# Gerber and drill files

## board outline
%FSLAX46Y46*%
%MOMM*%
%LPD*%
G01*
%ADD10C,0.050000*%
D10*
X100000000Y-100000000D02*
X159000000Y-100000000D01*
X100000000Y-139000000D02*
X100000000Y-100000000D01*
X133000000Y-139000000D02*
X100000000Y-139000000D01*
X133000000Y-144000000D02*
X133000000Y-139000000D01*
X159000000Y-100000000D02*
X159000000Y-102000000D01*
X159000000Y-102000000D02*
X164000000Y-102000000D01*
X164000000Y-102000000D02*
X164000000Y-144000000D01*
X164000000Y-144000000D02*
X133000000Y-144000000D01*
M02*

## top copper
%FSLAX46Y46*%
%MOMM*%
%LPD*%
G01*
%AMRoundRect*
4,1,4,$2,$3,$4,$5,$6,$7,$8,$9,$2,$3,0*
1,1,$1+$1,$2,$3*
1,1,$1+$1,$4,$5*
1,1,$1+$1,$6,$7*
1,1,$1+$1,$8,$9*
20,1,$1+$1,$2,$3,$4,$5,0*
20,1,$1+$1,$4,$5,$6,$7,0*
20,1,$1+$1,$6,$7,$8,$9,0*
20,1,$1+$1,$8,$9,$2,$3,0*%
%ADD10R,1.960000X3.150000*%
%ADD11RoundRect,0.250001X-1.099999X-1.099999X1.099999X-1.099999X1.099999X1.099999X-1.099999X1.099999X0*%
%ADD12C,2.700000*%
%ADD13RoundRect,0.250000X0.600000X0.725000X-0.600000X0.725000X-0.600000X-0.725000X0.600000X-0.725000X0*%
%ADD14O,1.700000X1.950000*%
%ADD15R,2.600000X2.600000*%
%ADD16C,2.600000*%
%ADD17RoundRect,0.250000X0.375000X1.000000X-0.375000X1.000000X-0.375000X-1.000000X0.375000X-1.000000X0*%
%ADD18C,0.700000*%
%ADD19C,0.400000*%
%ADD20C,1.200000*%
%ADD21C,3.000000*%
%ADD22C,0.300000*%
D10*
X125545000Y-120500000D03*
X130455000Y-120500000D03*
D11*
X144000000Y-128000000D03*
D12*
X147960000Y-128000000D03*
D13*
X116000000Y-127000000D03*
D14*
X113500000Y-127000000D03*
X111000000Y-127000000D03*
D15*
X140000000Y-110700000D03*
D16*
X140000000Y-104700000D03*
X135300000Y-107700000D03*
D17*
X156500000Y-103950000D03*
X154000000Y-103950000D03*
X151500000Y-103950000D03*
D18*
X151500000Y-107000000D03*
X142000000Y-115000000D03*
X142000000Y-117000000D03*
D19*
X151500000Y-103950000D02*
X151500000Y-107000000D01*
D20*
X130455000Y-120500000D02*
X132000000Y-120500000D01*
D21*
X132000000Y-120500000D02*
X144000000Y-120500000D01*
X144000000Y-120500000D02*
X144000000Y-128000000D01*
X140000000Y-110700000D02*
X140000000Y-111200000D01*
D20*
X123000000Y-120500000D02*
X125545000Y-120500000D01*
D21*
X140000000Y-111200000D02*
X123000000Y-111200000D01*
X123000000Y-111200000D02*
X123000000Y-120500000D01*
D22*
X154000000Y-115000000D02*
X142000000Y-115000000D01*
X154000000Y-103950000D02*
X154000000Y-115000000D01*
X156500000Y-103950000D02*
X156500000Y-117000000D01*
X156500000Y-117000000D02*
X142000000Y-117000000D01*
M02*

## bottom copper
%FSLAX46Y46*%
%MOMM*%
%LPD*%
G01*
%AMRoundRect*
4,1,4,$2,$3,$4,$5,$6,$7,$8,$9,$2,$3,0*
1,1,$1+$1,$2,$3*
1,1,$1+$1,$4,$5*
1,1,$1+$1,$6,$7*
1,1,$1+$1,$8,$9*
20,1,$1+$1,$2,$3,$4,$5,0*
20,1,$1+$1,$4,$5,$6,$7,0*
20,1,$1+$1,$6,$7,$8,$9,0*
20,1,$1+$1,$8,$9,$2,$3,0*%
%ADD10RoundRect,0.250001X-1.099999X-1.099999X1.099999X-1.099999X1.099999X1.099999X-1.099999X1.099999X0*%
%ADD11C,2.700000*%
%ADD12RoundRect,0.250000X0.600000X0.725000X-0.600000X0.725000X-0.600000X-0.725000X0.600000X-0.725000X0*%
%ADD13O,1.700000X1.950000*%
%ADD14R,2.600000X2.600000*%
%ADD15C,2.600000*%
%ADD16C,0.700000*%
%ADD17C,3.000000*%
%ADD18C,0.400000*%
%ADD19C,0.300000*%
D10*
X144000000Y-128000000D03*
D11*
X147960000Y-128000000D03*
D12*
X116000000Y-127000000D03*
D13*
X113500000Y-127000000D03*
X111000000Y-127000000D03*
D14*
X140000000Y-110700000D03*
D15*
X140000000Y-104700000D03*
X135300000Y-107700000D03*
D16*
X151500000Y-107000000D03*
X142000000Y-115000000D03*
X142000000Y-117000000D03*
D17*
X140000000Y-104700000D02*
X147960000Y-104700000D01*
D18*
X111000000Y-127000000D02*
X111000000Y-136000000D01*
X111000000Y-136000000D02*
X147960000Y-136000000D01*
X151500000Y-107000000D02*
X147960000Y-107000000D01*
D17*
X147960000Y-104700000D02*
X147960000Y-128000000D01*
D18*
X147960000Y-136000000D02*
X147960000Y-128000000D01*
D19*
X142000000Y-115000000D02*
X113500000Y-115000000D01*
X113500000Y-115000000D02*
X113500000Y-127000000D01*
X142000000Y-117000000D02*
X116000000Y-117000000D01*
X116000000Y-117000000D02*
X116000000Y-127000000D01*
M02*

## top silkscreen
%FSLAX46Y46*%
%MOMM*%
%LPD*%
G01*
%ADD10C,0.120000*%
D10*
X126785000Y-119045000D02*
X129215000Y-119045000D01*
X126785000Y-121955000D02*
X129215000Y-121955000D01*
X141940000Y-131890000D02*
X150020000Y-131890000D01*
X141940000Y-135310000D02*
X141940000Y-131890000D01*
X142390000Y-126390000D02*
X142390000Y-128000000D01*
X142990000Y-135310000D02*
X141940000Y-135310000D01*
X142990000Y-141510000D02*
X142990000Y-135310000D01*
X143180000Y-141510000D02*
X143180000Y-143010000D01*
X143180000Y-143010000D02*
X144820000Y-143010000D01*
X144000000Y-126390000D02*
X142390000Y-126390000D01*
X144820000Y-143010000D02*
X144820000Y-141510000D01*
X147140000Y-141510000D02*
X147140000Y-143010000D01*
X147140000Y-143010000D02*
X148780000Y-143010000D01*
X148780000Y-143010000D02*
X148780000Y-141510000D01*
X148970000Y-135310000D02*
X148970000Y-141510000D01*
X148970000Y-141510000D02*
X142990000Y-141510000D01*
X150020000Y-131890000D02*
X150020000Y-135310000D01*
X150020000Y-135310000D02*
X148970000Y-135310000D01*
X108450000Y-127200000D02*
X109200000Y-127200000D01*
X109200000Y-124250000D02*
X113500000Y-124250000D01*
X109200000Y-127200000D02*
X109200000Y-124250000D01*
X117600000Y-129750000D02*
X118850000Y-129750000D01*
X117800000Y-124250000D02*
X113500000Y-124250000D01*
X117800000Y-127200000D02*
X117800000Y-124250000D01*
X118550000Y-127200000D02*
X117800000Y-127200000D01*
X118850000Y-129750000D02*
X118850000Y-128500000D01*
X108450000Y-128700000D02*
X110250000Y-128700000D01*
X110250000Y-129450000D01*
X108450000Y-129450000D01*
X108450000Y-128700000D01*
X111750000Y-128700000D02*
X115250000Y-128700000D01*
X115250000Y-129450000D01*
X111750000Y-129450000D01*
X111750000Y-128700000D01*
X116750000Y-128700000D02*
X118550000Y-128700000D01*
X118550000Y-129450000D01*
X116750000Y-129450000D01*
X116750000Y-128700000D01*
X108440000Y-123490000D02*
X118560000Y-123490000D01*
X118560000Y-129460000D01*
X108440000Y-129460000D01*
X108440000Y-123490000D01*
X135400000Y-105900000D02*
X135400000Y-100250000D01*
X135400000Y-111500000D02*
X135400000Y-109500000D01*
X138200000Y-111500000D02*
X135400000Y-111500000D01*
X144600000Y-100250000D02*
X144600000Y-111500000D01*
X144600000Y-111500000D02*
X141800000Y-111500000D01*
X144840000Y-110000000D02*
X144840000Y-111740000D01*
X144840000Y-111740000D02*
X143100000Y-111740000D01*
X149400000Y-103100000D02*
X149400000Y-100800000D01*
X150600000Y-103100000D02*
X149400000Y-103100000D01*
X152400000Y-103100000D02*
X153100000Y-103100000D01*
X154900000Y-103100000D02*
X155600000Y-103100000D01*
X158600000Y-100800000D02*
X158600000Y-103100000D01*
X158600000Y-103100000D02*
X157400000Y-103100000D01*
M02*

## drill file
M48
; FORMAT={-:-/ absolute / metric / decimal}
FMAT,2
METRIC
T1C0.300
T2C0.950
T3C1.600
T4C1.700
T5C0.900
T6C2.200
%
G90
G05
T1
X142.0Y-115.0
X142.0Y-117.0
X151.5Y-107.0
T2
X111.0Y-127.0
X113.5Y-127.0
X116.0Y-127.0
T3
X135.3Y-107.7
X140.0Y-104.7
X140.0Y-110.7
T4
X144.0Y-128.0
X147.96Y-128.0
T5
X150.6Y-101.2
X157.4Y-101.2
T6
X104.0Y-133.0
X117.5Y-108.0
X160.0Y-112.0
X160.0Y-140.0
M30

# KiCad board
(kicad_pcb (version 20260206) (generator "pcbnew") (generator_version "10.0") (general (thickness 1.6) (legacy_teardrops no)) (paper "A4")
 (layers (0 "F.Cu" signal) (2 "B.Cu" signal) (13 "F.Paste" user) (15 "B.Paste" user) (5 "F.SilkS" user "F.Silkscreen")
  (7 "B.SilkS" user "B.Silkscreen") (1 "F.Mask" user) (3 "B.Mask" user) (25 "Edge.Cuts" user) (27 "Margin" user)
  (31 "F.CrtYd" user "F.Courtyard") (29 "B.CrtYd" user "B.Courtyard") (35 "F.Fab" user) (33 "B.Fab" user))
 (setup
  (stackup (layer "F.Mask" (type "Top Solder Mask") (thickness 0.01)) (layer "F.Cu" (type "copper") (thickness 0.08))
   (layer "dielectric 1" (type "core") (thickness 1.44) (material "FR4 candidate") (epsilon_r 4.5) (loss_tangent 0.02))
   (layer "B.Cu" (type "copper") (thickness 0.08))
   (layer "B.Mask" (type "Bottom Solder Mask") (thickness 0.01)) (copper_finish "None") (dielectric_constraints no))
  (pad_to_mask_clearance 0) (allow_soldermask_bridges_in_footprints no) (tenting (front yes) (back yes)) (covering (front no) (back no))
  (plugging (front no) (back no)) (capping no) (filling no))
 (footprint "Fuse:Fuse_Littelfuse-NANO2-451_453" (layer "F.Cu") (at 128 120.5)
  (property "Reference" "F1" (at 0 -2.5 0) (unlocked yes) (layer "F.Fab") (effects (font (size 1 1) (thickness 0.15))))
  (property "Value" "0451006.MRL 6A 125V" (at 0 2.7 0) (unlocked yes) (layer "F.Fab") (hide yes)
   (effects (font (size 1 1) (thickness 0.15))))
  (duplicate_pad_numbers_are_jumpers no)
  (fp_line (start -1.215 -1.455) (end 1.215 -1.455) (stroke (width 0.12) (type solid)) (layer "F.SilkS"))
  (fp_line (start -1.215 1.455) (end 1.215 1.455) (stroke (width 0.12) (type solid)) (layer "F.SilkS"))
  (pad "1" smd rect (at -2.455 0) (size 1.96 3.15) (layers "F.Cu" "F.Mask" "F.Paste") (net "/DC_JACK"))
  (pad "2" smd rect (at 2.455 0) (size 1.96 3.15) (layers "F.Cu" "F.Mask" "F.Paste") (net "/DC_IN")))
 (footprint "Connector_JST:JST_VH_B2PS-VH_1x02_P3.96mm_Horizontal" (layer "F.Cu") (at 144 128)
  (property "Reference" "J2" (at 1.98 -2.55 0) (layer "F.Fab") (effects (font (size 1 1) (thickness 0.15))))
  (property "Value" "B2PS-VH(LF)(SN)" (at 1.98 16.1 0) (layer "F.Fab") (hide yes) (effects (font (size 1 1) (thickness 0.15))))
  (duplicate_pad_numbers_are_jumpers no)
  (fp_line (start -2.06 3.89) (end 6.02 3.89) (stroke (width 0.12) (type solid)) (layer "F.SilkS"))
  (fp_line (start -2.06 7.31) (end -2.06 3.89) (stroke (width 0.12) (type solid)) (layer "F.SilkS"))
  (fp_line (start -1.61 -1.61) (end -1.61 0) (stroke (width 0.12) (type solid)) (layer "F.SilkS"))
  (fp_line (start -1.01 7.31) (end -2.06 7.31) (stroke (width 0.12) (type solid)) (layer "F.SilkS"))
  (fp_line (start -1.01 13.51) (end -1.01 7.31) (stroke (width 0.12) (type solid)) (layer "F.SilkS"))
  (fp_line (start -0.82 13.51) (end -0.82 15.01) (stroke (width 0.12) (type solid)) (layer "F.SilkS"))
  (fp_line (start -0.82 15.01) (end 0.82 15.01) (stroke (width 0.12) (type solid)) (layer "F.SilkS"))
  (fp_line (start 0 -1.61) (end -1.61 -1.61) (stroke (width 0.12) (type solid)) (layer "F.SilkS"))
  (fp_line (start 0.82 15.01) (end 0.82 13.51) (stroke (width 0.12) (type solid)) (layer "F.SilkS"))
  (fp_line (start 3.14 13.51) (end 3.14 15.01) (stroke (width 0.12) (type solid)) (layer "F.SilkS"))
  (fp_line (start 3.14 15.01) (end 4.78 15.01) (stroke (width 0.12) (type solid)) (layer "F.SilkS"))
  (fp_line (start 4.78 15.01) (end 4.78 13.51) (stroke (width 0.12) (type solid)) (layer "F.SilkS"))
  (fp_line (start 4.97 7.31) (end 4.97 13.51) (stroke (width 0.12) (type solid)) (layer "F.SilkS"))
  (fp_line (start 4.97 13.51) (end -1.01 13.51) (stroke (width 0.12) (type solid)) (layer "F.SilkS"))
  (fp_line (start 6.02 3.89) (end 6.02 7.31) (stroke (width 0.12) (type solid)) (layer "F.SilkS"))
  (fp_line (start 6.02 7.31) (end 4.97 7.31) (stroke (width 0.12) (type solid)) (layer "F.SilkS"))
  (pad "1" thru_hole roundrect (at 0 0) (size 2.7 2.7) (drill 1.7) (layers "*.Cu" "*.Mask") (remove_unused_layers no)
   (roundrect_rratio 0.092593) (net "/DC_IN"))
  (pad "2" thru_hole circle (at 3.96 0) (size 2.7 2.7) (drill 1.7) (layers "*.Cu" "*.Mask") (remove_unused_layers no) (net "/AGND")))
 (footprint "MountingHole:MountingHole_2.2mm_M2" (layer "F.Cu") (at 104 133)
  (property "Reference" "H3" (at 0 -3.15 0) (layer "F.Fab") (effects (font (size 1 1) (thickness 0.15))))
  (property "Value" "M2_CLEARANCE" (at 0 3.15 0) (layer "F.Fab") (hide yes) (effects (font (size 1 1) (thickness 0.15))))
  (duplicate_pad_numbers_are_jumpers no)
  (pad "" np_thru_hole circle (at 0 0) (size 2.2 2.2) (drill 2.2) (layers "*.Cu" "*.Mask")))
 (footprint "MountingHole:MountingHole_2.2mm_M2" (layer "F.Cu") (at 160 112)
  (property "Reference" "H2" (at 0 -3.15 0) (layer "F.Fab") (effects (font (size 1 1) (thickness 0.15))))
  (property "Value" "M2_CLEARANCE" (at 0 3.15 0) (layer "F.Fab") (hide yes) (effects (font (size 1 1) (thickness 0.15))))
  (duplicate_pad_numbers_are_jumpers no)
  (pad "" np_thru_hole circle (at 0 0) (size 2.2 2.2) (drill 2.2) (layers "*.Cu" "*.Mask")))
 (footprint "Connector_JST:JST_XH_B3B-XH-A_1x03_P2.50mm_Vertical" (layer "F.Cu") (at 116 127 180)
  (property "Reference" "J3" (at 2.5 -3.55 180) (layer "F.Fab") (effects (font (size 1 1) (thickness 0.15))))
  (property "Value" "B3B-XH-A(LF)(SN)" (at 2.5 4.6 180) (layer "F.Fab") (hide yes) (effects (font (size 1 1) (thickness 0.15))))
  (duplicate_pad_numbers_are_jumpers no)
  (fp_line (start 7.55 -0.2) (end 6.8 -0.2) (stroke (width 0.12) (type solid)) (layer "F.SilkS"))
  (fp_line (start 6.8 2.75) (end 2.5 2.75) (stroke (width 0.12) (type solid)) (layer "F.SilkS"))
  (fp_line (start 6.8 -0.2) (end 6.8 2.75) (stroke (width 0.12) (type solid)) (layer "F.SilkS"))
  (fp_line (start -1.6 -2.75) (end -2.85 -2.75) (stroke (width 0.12) (type solid)) (layer "F.SilkS"))
  (fp_line (start -1.8 2.75) (end 2.5 2.75) (stroke (width 0.12) (type solid)) (layer "F.SilkS"))
  (fp_line (start -1.8 -0.2) (end -1.8 2.75) (stroke (width 0.12) (type solid)) (layer "F.SilkS"))
  (fp_line (start -2.55 -0.2) (end -1.8 -0.2) (stroke (width 0.12) (type solid)) (layer "F.SilkS"))
  (fp_line (start -2.85 -2.75) (end -2.85 -1.5) (stroke (width 0.12) (type solid)) (layer "F.SilkS"))
  (fp_rect (start 5.75 -2.45) (end 7.55 -1.7) (stroke (width 0.12) (type solid)) (fill no) (layer "F.SilkS"))
  (fp_rect (start 0.75 -2.45) (end 4.25 -1.7) (stroke (width 0.12) (type solid)) (fill no) (layer "F.SilkS"))
  (fp_rect (start -2.55 -2.45) (end -0.75 -1.7) (stroke (width 0.12) (type solid)) (fill no) (layer "F.SilkS"))
  (fp_rect (start -2.56 -2.46) (end 7.56 3.51) (stroke (width 0.12) (type solid)) (fill no) (layer "F.SilkS"))
  (pad "1" thru_hole roundrect (at 0 0 180) (size 1.7 1.95) (drill 0.95) (layers "*.Cu" "*.Mask") (remove_unused_layers no)
   (roundrect_rratio 0.147059) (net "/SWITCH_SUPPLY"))
  (pad "2" thru_hole oval (at 2.5 0 180) (size 1.7 1.95) (drill 0.95) (layers "*.Cu" "*.Mask") (remove_unused_layers no) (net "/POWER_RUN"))
  (pad "3" thru_hole oval (at 5 0 180) (size 1.7 1.95) (drill 0.95) (layers "*.Cu" "*.Mask") (remove_unused_layers no) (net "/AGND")))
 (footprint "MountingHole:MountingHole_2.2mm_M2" (layer "F.Cu") (at 160 140)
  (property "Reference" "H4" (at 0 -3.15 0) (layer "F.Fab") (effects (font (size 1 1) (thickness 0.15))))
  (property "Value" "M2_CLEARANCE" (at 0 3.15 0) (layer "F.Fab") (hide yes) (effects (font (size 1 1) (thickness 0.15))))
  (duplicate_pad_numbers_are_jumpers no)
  (pad "" np_thru_hole circle (at 0 0) (size 2.2 2.2) (drill 2.2) (layers "*.Cu" "*.Mask")))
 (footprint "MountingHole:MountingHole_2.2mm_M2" (layer "F.Cu") (at 117.5 108)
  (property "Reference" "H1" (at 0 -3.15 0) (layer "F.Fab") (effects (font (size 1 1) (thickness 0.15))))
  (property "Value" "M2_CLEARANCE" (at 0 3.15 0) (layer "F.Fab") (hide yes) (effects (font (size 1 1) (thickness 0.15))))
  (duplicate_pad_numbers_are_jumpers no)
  (pad "" np_thru_hole circle (at 0 0) (size 2.2 2.2) (drill 2.2) (layers "*.Cu" "*.Mask")))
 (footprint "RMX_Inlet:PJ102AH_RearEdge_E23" (layer "F.Cu") (at 140 110.7 180)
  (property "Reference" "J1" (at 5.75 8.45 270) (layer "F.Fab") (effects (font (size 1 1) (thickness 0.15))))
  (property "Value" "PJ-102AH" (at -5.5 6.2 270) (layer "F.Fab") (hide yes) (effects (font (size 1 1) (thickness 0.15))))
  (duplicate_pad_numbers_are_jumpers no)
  (fp_line (start 4.6 4.8) (end 4.6 10.45) (stroke (width 0.12) (type solid)) (layer "F.SilkS"))
  (fp_line (start 4.6 -0.8) (end 4.6 1.2) (stroke (width 0.12) (type solid)) (layer "F.SilkS"))
  (fp_line (start 1.8 -0.8) (end 4.6 -0.8) (stroke (width 0.12) (type solid)) (layer "F.SilkS"))
  (fp_line (start -4.6 10.45) (end -4.6 -0.8) (stroke (width 0.12) (type solid)) (layer "F.SilkS"))
  (fp_line (start -4.6 -0.8) (end -1.8 -0.8) (stroke (width 0.12) (type solid)) (layer "F.SilkS"))
  (fp_line (start -4.84 0.7) (end -4.84 -1.04) (stroke (width 0.12) (type solid)) (layer "F.SilkS"))
  (fp_line (start -4.84 -1.04) (end -3.1 -1.04) (stroke (width 0.12) (type solid)) (layer "F.SilkS"))
  (pad "1" thru_hole rect (at 0 0 180) (size 2.6 2.6) (drill 1.6) (layers "*.Cu" "*.Mask") (remove_unused_layers no) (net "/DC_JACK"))
  (pad "2" thru_hole circle (at 0 6 180) (size 2.6 2.6) (drill 1.6) (layers "*.Cu" "*.Mask") (remove_unused_layers no) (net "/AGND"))
  (pad "3" thru_hole circle (at 4.7 3 180) (size 2.6 2.6) (drill 1.6) (layers "*.Cu" "*.Mask") (remove_unused_layers no)
   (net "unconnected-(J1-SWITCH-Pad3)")))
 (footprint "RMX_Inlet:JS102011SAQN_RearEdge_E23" (layer "F.Cu") (at 154 101.2 180)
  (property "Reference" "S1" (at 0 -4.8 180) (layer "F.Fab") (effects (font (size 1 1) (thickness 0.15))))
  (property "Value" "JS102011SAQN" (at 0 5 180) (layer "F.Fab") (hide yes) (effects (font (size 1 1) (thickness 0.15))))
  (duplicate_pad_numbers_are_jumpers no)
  (fp_line (start 4.6 -1.9) (end 4.6 0.4) (stroke (width 0.12) (type solid)) (layer "F.SilkS"))
  (fp_line (start 3.4 -1.9) (end 4.6 -1.9) (stroke (width 0.12) (type solid)) (layer "F.SilkS"))
  (fp_line (start 1.6 -1.9) (end 0.9 -1.9) (stroke (width 0.12) (type solid)) (layer "F.SilkS"))
  (fp_line (start -0.9 -1.9) (end -1.6 -1.9) (stroke (width 0.12) (type solid)) (layer "F.SilkS"))
  (fp_line (start -4.6 0.4) (end -4.6 -1.9) (stroke (width 0.12) (type solid)) (layer "F.SilkS"))
  (fp_line (start -4.6 -1.9) (end -3.4 -1.9) (stroke (width 0.12) (type solid)) (layer "F.SilkS"))
  (pad "" np_thru_hole circle (at -3.4 0 180) (size 0.9 0.9) (drill 0.9) (layers "*.Cu" "*.Mask"))
  (pad "" np_thru_hole circle (at 3.4 0 180) (size 0.9 0.9) (drill 0.9) (layers "*.Cu" "*.Mask"))
  (pad "1" smd roundrect (at -2.5 -2.75 180) (size 1.25 2.5) (layers "F.Cu" "F.Mask" "F.Paste") (roundrect_rratio 0.2)
   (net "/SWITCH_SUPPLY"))
  (pad "2" smd roundrect (at 0 -2.75 180) (size 1.25 2.5) (layers "F.Cu" "F.Mask" "F.Paste") (roundrect_rratio 0.2) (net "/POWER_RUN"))
  (pad "3" smd roundrect (at 2.5 -2.75 180) (size 1.25 2.5) (layers "F.Cu" "F.Mask" "F.Paste") (roundrect_rratio 0.2) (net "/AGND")))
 (gr_line (start 100 100) (end 159 100) (stroke (width 0.05) (type default)) (layer "Edge.Cuts"))
 (gr_line (start 100 139) (end 100 100) (stroke (width 0.05) (type default)) (layer "Edge.Cuts"))
 (gr_line (start 133 139) (end 100 139) (stroke (width 0.05) (type default)) (layer "Edge.Cuts"))
 (gr_line (start 133 144) (end 133 139) (stroke (width 0.05) (type default)) (layer "Edge.Cuts"))
 (gr_line (start 159 100) (end 159 102) (stroke (width 0.05) (type default)) (layer "Edge.Cuts"))
 (gr_line (start 159 102) (end 164 102) (stroke (width 0.05) (type default)) (layer "Edge.Cuts"))
 (gr_line (start 164 102) (end 164 144) (stroke (width 0.05) (type default)) (layer "Edge.Cuts"))
 (gr_line (start 164 144) (end 133 144) (stroke (width 0.05) (type default)) (layer "Edge.Cuts"))
 (segment (start 151.5 103.95) (end 151.5 107) (width 0.4) (layer "F.Cu") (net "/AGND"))
 (via (at 151.5 107) (size 0.7) (drill 0.3) (layers "F.Cu" "B.Cu") (capping no) (covering (front no) (back no))
  (plugging (front no) (back no)) (filling no) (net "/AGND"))
 (segment (start 140 104.7) (end 147.96 104.7) (width 3) (layer "B.Cu") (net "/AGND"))
 (segment (start 111 127) (end 111 136) (width 0.4) (layer "B.Cu") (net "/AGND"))
 (segment (start 111 136) (end 147.96 136) (width 0.4) (layer "B.Cu") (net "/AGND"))
 (segment (start 151.5 107) (end 147.96 107) (width 0.4) (layer "B.Cu") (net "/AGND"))
 (segment (start 147.96 104.7) (end 147.96 128) (width 3) (layer "B.Cu") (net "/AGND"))
 (segment (start 147.96 136) (end 147.96 128) (width 0.4) (layer "B.Cu") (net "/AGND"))
 (segment (start 130.455 120.5) (end 132 120.5) (width 1.2) (layer "F.Cu") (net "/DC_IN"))
 (segment (start 132 120.5) (end 144 120.5) (width 3) (layer "F.Cu") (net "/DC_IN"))
 (segment (start 144 120.5) (end 144 128) (width 3) (layer "F.Cu") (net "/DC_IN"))
 (segment (start 140 110.7) (end 140 111.2) (width 3) (layer "F.Cu") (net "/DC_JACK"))
 (segment (start 123 120.5) (end 125.545 120.5) (width 1.2) (layer "F.Cu") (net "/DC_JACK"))
 (segment (start 140 111.2) (end 123 111.2) (width 3) (layer "F.Cu") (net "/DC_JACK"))
 (segment (start 123 111.2) (end 123 120.5) (width 3) (layer "F.Cu") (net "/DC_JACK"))
 (segment (start 154 115) (end 142 115) (width 0.3) (layer "F.Cu") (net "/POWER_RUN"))
 (segment (start 154 103.95) (end 154 115) (width 0.3) (layer "F.Cu") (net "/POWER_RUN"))
 (via (at 142 115) (size 0.7) (drill 0.3) (layers "F.Cu" "B.Cu") (capping no) (covering (front no) (back no))
  (plugging (front no) (back no)) (filling no) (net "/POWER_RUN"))
 (segment (start 142 115) (end 113.5 115) (width 0.3) (layer "B.Cu") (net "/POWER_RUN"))
 (segment (start 113.5 115) (end 113.5 127) (width 0.3) (layer "B.Cu") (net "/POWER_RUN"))
 (segment (start 156.5 103.95) (end 156.5 117) (width 0.3) (layer "F.Cu") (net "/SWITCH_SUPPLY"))
 (segment (start 156.5 117) (end 142 117) (width 0.3) (layer "F.Cu") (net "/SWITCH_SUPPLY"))
 (via (at 142 117) (size 0.7) (drill 0.3) (layers "F.Cu" "B.Cu") (capping no) (covering (front no) (back no))
  (plugging (front no) (back no)) (filling no) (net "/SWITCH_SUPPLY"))
 (segment (start 142 117) (end 116 117) (width 0.3) (layer "B.Cu") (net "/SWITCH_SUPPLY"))
 (segment (start 116 117) (end 116 127) (width 0.3) (layer "B.Cu") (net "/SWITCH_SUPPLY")))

